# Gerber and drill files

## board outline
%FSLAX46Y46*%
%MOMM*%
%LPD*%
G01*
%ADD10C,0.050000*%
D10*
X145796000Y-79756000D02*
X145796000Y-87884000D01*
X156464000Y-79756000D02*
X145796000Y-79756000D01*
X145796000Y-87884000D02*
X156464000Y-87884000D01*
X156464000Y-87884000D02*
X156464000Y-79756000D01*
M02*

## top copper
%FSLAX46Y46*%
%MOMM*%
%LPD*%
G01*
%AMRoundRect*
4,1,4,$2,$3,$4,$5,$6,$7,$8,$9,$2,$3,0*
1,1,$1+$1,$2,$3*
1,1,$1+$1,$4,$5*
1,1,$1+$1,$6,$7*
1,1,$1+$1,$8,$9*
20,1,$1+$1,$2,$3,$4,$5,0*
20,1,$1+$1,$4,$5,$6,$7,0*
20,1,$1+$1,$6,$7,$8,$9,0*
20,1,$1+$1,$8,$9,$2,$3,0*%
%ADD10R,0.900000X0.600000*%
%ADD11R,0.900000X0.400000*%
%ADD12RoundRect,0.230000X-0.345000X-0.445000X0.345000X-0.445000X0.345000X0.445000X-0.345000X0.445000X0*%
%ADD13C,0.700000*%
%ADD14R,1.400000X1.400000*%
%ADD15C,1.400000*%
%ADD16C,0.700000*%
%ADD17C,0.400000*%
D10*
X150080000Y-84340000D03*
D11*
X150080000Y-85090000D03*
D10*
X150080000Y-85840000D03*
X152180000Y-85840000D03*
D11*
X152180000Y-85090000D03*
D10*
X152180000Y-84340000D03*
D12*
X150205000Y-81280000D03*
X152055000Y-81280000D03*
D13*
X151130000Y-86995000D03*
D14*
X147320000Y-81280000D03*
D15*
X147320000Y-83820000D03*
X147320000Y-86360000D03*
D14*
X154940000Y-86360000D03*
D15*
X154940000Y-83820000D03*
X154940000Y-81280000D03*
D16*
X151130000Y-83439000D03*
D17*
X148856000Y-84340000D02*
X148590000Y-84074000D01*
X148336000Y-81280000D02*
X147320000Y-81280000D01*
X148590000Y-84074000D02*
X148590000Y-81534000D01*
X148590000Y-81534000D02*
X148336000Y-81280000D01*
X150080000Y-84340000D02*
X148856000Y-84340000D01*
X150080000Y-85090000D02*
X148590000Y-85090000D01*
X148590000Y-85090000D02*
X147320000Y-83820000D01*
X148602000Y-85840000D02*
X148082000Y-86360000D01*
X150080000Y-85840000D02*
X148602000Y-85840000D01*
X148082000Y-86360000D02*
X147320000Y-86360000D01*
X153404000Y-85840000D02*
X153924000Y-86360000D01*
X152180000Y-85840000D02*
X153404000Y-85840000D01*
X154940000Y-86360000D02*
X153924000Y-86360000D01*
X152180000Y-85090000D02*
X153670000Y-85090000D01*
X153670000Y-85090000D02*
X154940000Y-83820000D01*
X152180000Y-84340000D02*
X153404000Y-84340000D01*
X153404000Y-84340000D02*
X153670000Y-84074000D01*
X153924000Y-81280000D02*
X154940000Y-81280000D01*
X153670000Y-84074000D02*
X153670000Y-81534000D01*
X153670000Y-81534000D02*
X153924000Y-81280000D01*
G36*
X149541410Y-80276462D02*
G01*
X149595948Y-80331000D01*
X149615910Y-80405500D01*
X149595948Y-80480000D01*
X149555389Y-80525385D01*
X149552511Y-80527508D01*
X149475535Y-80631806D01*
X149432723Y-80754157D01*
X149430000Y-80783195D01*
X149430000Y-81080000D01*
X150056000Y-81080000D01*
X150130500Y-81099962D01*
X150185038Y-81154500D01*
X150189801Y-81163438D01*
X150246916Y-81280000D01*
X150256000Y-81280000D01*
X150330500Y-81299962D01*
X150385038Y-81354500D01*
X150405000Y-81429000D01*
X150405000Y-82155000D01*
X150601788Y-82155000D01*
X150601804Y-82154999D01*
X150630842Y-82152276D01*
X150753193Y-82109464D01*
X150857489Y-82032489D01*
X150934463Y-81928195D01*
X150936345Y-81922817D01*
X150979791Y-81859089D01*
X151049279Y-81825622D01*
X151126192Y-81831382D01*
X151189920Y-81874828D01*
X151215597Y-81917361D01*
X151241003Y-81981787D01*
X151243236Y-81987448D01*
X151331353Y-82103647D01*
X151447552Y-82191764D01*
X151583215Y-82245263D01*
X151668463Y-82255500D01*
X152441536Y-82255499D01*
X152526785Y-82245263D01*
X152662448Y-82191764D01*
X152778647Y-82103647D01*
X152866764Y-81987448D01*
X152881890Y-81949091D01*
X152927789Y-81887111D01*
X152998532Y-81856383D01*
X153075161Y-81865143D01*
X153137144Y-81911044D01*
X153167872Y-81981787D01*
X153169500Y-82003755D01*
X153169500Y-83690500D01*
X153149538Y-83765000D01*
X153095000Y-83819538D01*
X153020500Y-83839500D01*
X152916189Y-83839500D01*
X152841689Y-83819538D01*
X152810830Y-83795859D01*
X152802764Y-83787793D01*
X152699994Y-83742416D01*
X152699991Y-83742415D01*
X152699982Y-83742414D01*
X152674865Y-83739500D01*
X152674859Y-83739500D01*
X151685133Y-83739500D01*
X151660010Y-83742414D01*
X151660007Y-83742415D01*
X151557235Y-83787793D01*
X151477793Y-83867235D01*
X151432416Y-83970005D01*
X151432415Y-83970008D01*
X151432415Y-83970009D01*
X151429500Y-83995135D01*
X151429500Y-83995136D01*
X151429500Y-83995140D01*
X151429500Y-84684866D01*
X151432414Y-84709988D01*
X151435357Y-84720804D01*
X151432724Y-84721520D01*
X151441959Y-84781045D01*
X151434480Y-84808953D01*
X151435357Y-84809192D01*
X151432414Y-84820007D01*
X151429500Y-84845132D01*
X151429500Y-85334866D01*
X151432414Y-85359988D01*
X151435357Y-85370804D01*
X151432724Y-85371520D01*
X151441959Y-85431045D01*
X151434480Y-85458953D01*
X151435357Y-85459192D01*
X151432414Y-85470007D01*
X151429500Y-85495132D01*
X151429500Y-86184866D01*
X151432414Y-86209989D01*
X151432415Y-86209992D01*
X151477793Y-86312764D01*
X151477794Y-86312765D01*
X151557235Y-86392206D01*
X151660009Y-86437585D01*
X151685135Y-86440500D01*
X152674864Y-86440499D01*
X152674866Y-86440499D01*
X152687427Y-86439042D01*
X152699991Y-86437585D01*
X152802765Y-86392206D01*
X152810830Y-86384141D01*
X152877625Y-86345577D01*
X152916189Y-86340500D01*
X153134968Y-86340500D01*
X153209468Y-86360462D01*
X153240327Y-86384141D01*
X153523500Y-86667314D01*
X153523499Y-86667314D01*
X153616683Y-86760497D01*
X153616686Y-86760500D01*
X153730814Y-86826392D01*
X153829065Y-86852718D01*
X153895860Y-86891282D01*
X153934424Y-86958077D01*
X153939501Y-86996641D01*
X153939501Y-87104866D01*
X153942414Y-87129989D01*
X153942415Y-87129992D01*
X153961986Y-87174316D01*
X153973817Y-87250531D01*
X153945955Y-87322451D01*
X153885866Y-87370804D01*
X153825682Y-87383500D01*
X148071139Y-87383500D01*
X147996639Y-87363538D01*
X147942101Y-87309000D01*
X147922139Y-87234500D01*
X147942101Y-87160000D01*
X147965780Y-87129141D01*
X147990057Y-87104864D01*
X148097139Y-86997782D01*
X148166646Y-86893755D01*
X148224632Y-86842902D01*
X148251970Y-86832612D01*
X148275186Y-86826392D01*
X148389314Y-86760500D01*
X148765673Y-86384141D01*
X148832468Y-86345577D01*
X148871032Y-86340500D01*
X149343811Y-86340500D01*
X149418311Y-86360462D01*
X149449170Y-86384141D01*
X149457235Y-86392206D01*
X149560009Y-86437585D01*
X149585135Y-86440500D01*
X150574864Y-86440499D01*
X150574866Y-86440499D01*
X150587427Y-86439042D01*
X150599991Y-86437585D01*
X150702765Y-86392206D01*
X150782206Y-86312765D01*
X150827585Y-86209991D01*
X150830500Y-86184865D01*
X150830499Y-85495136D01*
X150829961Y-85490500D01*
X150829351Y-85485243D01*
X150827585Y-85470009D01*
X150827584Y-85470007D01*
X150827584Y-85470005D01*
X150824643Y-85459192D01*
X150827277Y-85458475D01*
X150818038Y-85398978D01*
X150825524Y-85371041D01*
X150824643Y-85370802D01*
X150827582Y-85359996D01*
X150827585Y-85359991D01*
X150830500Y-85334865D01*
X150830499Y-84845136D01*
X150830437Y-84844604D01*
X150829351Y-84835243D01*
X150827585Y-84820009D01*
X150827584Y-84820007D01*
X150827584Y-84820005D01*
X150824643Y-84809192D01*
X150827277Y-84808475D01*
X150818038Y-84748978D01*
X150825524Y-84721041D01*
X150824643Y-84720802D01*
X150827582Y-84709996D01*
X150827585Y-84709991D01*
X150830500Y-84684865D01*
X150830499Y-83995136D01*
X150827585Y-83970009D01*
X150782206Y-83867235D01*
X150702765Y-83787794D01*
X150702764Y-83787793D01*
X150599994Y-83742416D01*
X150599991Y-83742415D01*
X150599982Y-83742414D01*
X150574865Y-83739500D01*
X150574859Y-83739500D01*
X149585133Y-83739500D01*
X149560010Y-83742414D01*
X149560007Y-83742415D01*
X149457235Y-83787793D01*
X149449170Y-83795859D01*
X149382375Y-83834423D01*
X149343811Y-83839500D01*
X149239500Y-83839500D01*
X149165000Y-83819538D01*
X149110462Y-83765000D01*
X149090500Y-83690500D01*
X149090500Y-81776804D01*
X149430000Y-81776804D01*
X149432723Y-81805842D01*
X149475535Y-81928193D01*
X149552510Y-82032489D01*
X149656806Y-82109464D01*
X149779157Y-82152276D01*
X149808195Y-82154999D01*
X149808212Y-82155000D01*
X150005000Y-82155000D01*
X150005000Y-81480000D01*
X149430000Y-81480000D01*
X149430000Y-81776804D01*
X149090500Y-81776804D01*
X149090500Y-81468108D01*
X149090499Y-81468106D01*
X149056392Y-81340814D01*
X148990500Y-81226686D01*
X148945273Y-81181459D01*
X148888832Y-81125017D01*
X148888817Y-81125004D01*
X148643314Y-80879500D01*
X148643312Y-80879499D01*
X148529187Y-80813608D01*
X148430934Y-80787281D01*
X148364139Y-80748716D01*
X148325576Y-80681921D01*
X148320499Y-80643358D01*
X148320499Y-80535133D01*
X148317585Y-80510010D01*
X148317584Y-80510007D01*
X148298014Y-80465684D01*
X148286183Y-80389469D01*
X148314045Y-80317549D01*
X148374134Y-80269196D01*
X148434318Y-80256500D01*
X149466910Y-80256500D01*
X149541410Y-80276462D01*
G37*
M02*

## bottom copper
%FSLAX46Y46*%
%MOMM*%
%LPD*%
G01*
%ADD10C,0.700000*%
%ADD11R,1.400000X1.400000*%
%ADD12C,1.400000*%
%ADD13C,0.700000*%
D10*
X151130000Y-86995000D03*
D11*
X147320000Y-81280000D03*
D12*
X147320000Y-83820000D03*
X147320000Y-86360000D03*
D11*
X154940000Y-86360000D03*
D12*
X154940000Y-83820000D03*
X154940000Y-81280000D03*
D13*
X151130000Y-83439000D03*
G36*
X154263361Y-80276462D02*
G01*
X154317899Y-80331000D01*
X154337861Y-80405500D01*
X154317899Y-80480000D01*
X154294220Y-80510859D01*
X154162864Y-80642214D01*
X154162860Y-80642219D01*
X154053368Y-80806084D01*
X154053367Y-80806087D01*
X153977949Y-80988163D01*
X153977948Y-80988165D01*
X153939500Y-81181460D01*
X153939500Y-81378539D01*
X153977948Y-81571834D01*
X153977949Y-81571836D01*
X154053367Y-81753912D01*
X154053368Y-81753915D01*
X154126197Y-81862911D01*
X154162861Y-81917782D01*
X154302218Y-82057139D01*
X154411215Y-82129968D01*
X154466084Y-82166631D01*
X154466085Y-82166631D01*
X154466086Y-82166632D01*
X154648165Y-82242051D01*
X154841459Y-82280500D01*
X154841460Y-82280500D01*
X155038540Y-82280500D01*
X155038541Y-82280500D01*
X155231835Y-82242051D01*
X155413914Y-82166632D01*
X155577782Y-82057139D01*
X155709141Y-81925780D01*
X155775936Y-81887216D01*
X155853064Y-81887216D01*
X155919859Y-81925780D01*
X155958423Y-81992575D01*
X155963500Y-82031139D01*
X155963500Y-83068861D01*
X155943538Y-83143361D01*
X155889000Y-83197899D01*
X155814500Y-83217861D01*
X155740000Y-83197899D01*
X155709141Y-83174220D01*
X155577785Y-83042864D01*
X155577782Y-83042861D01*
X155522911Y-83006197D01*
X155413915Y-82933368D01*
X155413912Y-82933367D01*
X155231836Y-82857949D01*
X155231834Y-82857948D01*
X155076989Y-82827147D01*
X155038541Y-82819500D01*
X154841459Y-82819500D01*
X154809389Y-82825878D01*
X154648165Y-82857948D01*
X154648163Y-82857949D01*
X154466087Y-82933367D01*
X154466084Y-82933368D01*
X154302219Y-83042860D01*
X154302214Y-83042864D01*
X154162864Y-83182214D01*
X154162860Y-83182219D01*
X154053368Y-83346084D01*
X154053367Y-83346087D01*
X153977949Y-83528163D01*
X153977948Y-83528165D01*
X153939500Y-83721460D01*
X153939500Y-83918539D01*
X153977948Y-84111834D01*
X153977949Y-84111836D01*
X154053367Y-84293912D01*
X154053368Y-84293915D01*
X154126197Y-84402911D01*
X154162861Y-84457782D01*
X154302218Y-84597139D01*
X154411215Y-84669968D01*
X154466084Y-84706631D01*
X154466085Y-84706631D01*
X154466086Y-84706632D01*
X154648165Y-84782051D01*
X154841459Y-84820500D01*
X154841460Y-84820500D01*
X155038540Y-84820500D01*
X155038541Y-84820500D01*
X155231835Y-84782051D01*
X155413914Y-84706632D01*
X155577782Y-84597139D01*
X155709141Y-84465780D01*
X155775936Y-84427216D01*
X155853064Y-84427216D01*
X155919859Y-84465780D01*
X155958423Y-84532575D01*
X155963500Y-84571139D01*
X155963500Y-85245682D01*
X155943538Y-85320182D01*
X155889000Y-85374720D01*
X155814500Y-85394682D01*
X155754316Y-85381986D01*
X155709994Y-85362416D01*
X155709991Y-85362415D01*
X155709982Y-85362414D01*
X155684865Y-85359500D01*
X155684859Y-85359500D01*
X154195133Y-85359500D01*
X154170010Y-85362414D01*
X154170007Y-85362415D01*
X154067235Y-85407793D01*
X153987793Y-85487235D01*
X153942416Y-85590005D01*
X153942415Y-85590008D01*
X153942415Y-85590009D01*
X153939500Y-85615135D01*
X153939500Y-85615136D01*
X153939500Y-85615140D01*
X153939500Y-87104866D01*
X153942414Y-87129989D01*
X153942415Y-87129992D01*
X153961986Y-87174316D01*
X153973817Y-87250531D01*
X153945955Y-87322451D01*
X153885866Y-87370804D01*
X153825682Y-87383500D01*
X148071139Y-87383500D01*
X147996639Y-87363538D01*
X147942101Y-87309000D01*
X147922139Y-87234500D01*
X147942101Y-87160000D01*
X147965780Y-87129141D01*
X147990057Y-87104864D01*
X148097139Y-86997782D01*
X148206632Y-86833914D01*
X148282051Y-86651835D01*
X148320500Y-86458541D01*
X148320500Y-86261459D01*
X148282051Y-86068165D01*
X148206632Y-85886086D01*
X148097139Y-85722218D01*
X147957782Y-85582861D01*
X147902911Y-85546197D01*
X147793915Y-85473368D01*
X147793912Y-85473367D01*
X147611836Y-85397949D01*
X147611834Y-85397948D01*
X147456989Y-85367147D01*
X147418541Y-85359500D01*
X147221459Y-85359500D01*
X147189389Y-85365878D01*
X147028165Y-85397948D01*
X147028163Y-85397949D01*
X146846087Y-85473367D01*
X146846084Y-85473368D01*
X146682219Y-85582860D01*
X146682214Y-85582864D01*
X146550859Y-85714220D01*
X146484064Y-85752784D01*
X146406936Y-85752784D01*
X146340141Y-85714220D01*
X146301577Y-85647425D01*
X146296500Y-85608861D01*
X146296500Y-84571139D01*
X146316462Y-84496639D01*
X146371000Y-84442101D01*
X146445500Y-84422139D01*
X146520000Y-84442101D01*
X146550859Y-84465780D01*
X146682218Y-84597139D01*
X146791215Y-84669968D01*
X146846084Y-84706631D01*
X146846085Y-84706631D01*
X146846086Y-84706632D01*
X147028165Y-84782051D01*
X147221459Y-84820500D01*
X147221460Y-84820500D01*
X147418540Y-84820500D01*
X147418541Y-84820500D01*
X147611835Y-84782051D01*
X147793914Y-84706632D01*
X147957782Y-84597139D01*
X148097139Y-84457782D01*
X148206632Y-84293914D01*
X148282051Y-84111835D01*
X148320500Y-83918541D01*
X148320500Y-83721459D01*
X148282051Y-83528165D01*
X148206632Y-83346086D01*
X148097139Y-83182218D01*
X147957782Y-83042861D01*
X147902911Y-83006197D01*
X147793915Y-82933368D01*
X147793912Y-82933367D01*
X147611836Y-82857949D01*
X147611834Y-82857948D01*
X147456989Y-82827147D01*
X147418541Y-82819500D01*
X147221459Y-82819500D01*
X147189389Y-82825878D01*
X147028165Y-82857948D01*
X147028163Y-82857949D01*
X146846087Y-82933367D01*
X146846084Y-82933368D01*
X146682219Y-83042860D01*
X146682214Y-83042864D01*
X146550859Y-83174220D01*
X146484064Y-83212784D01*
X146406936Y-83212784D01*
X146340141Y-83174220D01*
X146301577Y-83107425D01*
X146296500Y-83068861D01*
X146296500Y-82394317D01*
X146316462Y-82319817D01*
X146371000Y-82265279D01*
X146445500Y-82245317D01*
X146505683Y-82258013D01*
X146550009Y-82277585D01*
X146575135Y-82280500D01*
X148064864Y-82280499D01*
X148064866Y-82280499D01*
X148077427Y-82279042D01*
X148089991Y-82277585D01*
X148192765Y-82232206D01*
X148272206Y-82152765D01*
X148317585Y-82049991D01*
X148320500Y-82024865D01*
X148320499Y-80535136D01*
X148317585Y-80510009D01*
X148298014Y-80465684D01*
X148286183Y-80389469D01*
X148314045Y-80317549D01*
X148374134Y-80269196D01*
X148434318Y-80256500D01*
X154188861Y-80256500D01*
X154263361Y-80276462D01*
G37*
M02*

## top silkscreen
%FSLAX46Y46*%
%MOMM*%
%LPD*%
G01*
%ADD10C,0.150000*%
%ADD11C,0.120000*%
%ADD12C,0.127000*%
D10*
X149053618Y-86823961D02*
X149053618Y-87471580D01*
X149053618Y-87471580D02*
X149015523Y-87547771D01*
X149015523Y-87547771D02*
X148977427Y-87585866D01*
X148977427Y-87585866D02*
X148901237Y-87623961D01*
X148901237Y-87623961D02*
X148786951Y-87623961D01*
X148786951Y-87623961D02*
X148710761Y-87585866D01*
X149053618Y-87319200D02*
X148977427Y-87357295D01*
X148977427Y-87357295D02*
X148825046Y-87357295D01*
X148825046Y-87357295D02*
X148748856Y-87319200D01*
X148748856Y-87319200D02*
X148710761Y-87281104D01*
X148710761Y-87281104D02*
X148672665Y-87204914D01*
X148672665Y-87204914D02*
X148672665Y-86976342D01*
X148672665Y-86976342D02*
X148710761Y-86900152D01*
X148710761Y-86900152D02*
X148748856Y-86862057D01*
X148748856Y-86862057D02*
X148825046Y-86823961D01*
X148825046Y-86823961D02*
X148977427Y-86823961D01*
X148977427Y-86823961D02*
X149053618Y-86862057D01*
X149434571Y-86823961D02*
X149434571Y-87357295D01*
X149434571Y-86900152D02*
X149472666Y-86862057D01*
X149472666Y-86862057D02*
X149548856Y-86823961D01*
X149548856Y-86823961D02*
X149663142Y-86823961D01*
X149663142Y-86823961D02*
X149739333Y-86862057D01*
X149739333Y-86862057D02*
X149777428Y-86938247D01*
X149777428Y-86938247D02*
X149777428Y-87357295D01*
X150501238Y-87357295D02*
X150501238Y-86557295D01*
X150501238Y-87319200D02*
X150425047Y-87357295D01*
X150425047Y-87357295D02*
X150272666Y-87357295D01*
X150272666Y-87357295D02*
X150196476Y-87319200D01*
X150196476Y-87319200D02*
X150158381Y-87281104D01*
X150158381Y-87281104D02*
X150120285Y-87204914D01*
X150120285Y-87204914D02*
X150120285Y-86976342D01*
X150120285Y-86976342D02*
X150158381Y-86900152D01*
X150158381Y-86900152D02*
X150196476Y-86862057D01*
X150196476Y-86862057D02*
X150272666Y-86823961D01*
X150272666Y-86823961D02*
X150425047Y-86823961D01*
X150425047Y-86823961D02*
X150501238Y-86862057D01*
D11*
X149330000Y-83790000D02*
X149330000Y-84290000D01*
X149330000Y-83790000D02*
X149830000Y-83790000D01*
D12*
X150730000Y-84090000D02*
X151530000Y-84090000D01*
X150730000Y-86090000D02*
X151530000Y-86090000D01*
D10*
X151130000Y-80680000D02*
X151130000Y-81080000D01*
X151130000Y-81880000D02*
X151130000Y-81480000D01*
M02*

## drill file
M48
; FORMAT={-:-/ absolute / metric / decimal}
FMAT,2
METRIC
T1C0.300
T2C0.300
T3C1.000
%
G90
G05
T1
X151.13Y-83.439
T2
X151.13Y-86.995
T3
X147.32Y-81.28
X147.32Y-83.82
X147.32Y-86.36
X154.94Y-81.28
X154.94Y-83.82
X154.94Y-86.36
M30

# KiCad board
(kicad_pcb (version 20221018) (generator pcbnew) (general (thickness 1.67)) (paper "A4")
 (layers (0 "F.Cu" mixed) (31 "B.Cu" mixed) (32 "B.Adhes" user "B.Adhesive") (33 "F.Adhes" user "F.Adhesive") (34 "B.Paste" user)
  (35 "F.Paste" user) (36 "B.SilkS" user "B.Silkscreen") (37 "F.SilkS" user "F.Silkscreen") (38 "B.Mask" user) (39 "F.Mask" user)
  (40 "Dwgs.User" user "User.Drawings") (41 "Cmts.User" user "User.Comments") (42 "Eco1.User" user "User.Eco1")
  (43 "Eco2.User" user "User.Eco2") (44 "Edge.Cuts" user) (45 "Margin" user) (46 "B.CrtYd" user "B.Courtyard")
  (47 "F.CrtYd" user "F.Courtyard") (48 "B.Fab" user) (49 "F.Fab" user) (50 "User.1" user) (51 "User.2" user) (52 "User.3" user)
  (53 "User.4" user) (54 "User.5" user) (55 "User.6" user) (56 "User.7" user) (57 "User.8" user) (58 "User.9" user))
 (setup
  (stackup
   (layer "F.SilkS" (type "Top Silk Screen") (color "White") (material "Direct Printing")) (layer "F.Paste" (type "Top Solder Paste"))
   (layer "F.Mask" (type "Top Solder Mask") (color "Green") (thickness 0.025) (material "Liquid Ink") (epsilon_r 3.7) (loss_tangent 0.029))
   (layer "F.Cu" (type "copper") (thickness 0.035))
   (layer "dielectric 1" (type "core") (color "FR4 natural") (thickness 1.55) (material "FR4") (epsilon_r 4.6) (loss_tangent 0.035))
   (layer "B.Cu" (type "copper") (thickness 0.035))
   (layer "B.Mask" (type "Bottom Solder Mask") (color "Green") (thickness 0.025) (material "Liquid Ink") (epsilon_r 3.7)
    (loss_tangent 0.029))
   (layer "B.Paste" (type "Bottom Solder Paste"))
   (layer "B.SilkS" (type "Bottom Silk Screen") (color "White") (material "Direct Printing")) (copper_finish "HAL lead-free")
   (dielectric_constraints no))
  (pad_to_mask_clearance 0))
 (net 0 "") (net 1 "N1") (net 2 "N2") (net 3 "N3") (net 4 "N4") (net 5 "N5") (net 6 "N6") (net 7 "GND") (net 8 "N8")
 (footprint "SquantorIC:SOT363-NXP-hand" (layer "F.Cu") (at 151.13 85.09)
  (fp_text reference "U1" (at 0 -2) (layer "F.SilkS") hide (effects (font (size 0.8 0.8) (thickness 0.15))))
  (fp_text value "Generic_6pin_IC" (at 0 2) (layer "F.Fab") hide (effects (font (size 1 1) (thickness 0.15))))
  (fp_line (start -1.8 -1.3) (end -1.8 -0.8) (stroke (width 0.12) (type solid)) (layer "F.SilkS"))
  (fp_line (start -1.8 -1.3) (end -1.3 -1.3) (stroke (width 0.12) (type solid)) (layer "F.SilkS"))
  (fp_line (start -0.4 -1) (end 0.4 -1) (stroke (width 0.127) (type solid)) (layer "F.SilkS"))
  (fp_line (start -0.4 1) (end 0.4 1) (stroke (width 0.127) (type solid)) (layer "F.SilkS"))
  (pad "1" smd rect (at -1.05 -0.75 270) (size 0.6 0.9) (layers "F.Cu" "F.Paste" "F.Mask") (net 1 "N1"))
  (pad "2" smd rect (at -1.05 0 270) (size 0.4 0.9) (layers "F.Cu" "F.Paste" "F.Mask") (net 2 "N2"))
  (pad "3" smd rect (at -1.05 0.75 270) (size 0.6 0.9) (layers "F.Cu" "F.Paste" "F.Mask") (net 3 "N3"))
  (pad "4" smd rect (at 1.05 0.75 270) (size 0.6 0.9) (layers "F.Cu" "F.Paste" "F.Mask") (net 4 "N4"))
  (pad "5" smd rect (at 1.05 0 270) (size 0.4 0.9) (layers "F.Cu" "F.Paste" "F.Mask") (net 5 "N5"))
  (pad "6" smd rect (at 1.05 -0.75 270) (size 0.6 0.9) (layers "F.Cu" "F.Paste" "F.Mask") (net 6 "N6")))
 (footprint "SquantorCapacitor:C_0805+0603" (layer "F.Cu") (at 151.13 81.28)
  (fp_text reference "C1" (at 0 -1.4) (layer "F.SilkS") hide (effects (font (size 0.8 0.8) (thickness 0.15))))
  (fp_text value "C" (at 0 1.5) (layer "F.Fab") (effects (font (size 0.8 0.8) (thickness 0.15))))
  (fp_line (start 0 -0.6) (end 0 -0.2) (stroke (width 0.15) (type solid)) (layer "F.SilkS"))
  (fp_line (start 0 0.6) (end 0 0.2) (stroke (width 0.15) (type solid)) (layer "F.SilkS"))
  (pad "1" smd roundrect (at -0.925 0) (size 1.15 1.35) (layers "F.Cu" "F.Paste" "F.Mask") (roundrect_rratio 0.2) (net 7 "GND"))
  (pad "2" smd roundrect (at 0.925 0) (size 1.15 1.35) (layers "F.Cu" "F.Paste" "F.Mask") (roundrect_rratio 0.2) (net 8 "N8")))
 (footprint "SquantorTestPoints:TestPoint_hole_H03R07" (layer "F.Cu") (at 151.13 86.995)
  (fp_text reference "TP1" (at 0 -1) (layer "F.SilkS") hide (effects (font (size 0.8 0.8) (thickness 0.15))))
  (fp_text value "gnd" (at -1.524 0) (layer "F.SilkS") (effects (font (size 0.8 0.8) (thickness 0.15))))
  (pad "1" thru_hole circle (at 0 0) (size 0.7 0.7) (drill 0.3) (layers "*.Cu" "*.Mask") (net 7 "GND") (zone_connect 2)))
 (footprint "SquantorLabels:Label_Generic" (layer "B.Cu") (at 151.3 83.4 -90)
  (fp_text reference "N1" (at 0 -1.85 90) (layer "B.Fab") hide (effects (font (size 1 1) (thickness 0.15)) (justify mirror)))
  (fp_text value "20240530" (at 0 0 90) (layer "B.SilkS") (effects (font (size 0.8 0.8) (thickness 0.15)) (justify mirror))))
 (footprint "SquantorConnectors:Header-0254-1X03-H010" (layer "B.Cu") (at 147.32 83.82 -90)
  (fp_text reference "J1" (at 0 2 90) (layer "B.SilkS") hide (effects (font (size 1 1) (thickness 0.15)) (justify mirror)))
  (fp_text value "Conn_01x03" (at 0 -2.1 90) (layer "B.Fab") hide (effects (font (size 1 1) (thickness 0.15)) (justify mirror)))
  (pad "1" thru_hole rect (at -2.54 0 90) (size 1.4 1.4) (drill 1) (layers "*.Cu" "*.Mask") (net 1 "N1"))
  (pad "2" thru_hole circle (at 0 0 90) (size 1.4 1.4) (drill 1) (layers "*.Cu" "*.Mask") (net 2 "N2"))
  (pad "3" thru_hole circle (at 2.54 0 90) (size 1.4 1.4) (drill 1) (layers "*.Cu" "*.Mask") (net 3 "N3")))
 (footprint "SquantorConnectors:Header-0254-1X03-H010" (layer "B.Cu") (at 154.94 83.82 90)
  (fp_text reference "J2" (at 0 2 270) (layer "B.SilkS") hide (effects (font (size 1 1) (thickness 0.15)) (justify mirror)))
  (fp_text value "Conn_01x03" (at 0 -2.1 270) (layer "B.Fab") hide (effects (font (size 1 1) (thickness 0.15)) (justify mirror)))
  (pad "1" thru_hole rect (at -2.54 0 270) (size 1.4 1.4) (drill 1) (layers "*.Cu" "*.Mask") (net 4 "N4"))
  (pad "2" thru_hole circle (at 0 0 270) (size 1.4 1.4) (drill 1) (layers "*.Cu" "*.Mask") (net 5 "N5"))
  (pad "3" thru_hole circle (at 2.54 0 270) (size 1.4 1.4) (drill 1) (layers "*.Cu" "*.Mask") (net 6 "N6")))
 (gr_line (start 145.796 79.756) (end 145.796 87.884) (stroke (width 0.05) (type solid)) (layer "Edge.Cuts"))
 (gr_line (start 156.464 79.756) (end 145.796 79.756) (stroke (width 0.05) (type solid)) (layer "Edge.Cuts"))
 (gr_line (start 145.796 87.884) (end 156.464 87.884) (stroke (width 0.05) (type solid)) (layer "Edge.Cuts"))
 (gr_line (start 156.464 87.884) (end 156.464 79.756) (stroke (width 0.05) (type solid)) (layer "Edge.Cuts"))
 (via (at 151.13 83.439) (size 0.7) (drill 0.3) (layers "F.Cu" "B.Cu") (free) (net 7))
 (segment (start 148.856 84.34) (end 148.59 84.074) (width 0.4) (layer "F.Cu") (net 1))
 (segment (start 148.336 81.28) (end 147.32 81.28) (width 0.4) (layer "F.Cu") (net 1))
 (segment (start 148.59 84.074) (end 148.59 81.534) (width 0.4) (layer "F.Cu") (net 1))
 (segment (start 148.59 81.534) (end 148.336 81.28) (width 0.4) (layer "F.Cu") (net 1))
 (segment (start 150.08 84.34) (end 148.856 84.34) (width 0.4) (layer "F.Cu") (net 1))
 (segment (start 150.08 85.09) (end 148.59 85.09) (width 0.4) (layer "F.Cu") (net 2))
 (segment (start 148.59 85.09) (end 147.32 83.82) (width 0.4) (layer "F.Cu") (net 2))
 (segment (start 148.602 85.84) (end 148.082 86.36) (width 0.4) (layer "F.Cu") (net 3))
 (segment (start 150.08 85.84) (end 148.602 85.84) (width 0.4) (layer "F.Cu") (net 3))
 (segment (start 148.082 86.36) (end 147.32 86.36) (width 0.4) (layer "F.Cu") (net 3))
 (segment (start 153.404 85.84) (end 153.924 86.36) (width 0.4) (layer "F.Cu") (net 4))
 (segment (start 152.18 85.84) (end 153.404 85.84) (width 0.4) (layer "F.Cu") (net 4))
 (segment (start 154.94 86.36) (end 153.924 86.36) (width 0.4) (layer "F.Cu") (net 4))
 (segment (start 152.18 85.09) (end 153.67 85.09) (width 0.4) (layer "F.Cu") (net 5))
 (segment (start 153.67 85.09) (end 154.94 83.82) (width 0.4) (layer "F.Cu") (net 5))
 (segment (start 152.18 84.34) (end 153.404 84.34) (width 0.4) (layer "F.Cu") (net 6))
 (segment (start 153.404 84.34) (end 153.67 84.074) (width 0.4) (layer "F.Cu") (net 6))
 (segment (start 153.924 81.28) (end 154.94 81.28) (width 0.4) (layer "F.Cu") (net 6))
 (segment (start 153.67 84.074) (end 153.67 81.534) (width 0.4) (layer "F.Cu") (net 6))
 (segment (start 153.67 81.534) (end 153.924 81.28) (width 0.4) (layer "F.Cu") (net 6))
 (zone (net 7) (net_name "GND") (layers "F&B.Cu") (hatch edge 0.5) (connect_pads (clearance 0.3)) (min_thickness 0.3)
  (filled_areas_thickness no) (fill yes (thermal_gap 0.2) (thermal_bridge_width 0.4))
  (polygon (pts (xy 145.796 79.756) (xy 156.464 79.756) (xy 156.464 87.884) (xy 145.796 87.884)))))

